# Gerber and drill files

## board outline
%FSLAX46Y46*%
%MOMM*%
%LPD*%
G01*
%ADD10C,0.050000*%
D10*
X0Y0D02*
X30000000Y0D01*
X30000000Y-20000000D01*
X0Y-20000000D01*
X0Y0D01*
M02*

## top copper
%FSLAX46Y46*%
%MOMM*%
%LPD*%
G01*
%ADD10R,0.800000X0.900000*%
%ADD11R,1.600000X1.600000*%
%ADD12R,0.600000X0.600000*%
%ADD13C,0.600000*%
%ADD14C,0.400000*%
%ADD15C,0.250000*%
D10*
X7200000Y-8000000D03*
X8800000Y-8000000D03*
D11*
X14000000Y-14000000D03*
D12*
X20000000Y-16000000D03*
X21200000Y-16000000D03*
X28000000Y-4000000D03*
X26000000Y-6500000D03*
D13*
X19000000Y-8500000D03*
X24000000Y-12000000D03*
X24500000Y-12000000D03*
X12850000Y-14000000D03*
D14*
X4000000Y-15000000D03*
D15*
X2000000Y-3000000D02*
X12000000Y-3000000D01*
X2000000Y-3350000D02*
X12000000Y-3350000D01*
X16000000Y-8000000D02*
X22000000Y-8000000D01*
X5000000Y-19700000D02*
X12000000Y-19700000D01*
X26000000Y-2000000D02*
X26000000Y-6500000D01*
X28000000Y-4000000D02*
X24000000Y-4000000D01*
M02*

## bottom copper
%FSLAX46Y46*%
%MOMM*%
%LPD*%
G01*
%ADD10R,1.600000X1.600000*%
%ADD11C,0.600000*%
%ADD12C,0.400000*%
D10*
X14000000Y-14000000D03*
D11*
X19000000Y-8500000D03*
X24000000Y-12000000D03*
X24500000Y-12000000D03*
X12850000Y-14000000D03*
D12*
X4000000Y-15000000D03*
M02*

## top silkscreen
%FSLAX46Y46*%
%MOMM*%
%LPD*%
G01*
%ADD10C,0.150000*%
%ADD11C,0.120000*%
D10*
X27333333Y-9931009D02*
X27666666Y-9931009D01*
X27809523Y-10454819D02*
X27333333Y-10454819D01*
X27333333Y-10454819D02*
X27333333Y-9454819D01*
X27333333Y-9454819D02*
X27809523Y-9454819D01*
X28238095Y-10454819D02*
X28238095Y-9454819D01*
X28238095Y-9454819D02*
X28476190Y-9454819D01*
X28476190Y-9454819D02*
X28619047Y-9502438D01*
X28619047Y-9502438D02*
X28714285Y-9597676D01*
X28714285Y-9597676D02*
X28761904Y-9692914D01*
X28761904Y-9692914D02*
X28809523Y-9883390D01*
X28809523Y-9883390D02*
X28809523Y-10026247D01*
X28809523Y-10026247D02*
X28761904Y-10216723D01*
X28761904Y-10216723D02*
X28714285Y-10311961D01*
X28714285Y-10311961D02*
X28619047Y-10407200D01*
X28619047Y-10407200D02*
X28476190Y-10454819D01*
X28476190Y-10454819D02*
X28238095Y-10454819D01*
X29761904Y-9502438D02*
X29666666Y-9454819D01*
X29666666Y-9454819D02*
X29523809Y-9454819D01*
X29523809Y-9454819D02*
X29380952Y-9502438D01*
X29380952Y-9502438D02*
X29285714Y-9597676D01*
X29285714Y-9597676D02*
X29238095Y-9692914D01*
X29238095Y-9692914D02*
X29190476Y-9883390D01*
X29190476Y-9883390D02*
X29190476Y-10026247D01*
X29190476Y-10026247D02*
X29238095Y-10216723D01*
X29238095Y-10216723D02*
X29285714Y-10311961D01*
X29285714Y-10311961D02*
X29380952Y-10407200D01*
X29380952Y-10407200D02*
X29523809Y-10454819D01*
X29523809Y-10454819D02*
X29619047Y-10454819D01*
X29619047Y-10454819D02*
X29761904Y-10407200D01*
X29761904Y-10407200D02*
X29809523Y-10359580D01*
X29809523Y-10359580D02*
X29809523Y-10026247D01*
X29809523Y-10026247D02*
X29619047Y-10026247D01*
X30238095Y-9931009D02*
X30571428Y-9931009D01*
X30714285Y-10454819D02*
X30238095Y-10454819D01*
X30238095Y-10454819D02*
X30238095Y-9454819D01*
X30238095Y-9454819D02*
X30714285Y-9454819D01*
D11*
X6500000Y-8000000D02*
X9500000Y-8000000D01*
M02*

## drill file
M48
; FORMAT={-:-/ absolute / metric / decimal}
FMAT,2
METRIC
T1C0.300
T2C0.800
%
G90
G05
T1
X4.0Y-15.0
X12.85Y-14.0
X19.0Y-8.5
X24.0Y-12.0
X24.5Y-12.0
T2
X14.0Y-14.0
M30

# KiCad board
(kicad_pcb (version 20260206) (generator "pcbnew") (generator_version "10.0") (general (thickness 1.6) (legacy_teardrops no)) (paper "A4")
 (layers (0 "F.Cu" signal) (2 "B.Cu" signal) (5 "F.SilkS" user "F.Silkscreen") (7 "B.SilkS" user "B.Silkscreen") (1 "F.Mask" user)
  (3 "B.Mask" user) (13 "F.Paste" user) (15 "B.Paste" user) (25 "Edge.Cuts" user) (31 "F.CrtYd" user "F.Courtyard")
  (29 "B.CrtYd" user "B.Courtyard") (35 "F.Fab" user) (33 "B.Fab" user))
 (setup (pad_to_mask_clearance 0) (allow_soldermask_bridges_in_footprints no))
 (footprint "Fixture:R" (layer "F.Cu") (at 8 8)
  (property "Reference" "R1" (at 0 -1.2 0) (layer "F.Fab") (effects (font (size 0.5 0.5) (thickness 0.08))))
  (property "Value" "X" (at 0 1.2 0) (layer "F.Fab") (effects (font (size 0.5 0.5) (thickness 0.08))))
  (pad "1" smd rect (at -0.8 0) (size 0.8 0.9) (layers "F.Cu" "F.Mask" "F.Paste") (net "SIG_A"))
  (pad "2" smd rect (at 0.8 0) (size 0.8 0.9) (layers "F.Cu" "F.Mask" "F.Paste") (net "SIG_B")))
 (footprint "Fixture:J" (layer "F.Cu") (at 14 14)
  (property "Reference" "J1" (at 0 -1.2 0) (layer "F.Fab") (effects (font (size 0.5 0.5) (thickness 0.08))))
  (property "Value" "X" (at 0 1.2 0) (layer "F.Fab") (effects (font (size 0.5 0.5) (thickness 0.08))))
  (pad "1" thru_hole rect (at 0 0) (size 1.6 1.6) (drill 0.8) (layers "*.Cu" "*.Mask") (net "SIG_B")))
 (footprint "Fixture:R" (layer "F.Cu") (at 20 16)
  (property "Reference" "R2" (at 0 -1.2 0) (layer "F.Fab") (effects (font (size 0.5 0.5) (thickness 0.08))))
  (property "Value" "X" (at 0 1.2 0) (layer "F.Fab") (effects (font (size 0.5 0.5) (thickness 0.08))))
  (pad "1" smd rect (at 0 0) (size 0.6 0.6) (layers "F.Cu" "F.Mask" "F.Paste")))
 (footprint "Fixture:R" (layer "F.Cu") (at 21.2 16)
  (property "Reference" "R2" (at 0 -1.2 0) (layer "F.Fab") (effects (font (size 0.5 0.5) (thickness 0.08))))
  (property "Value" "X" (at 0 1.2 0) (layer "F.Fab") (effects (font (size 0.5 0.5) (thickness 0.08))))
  (pad "1" smd rect (at 0 0) (size 0.6 0.6) (layers "F.Cu" "F.Mask" "F.Paste")))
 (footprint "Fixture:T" (layer "F.Cu") (at 28 4)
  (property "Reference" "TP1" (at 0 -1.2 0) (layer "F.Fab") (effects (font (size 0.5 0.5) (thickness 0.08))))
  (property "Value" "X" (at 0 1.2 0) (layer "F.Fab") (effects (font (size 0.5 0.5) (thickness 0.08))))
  (pad "1" smd rect (at 0 0) (size 0.6 0.6) (layers "F.Cu" "F.Mask" "F.Paste") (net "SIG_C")))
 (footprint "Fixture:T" (layer "F.Cu") (at 26 6.5)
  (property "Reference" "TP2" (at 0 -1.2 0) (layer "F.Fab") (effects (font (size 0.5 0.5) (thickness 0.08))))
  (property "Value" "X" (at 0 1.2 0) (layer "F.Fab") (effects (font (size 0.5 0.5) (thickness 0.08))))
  (pad "1" smd rect (at 0 0) (size 0.6 0.6) (layers "F.Cu" "F.Mask" "F.Paste") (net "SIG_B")))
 (gr_rect (start 0 0) (end 30 20) (stroke (width 0.05) (type default)) (fill no) (layer "Edge.Cuts"))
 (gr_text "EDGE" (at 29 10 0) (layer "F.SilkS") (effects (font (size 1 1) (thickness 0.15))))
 (gr_line (start 6.5 8) (end 9.5 8) (stroke (width 0.12) (type default)) (layer "F.SilkS"))
 (segment (start 2 3) (end 12 3) (width 0.25) (layer "F.Cu") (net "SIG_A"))
 (segment (start 2 3.35) (end 12 3.35) (width 0.25) (layer "F.Cu") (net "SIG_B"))
 (segment (start 16 8) (end 22 8) (width 0.25) (layer "F.Cu") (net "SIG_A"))
 (via (at 19 8.5) (size 0.6) (drill 0.3) (layers "F.Cu" "B.Cu") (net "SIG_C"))
 (via (at 24 12) (size 0.6) (drill 0.3) (layers "F.Cu" "B.Cu") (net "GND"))
 (via (at 24.5 12) (size 0.6) (drill 0.3) (layers "F.Cu" "B.Cu") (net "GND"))
 (segment (start 5 19.7) (end 12 19.7) (width 0.25) (layer "F.Cu") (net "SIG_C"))
 (segment (start 26 2) (end 26 6.5) (width 0.25) (layer "F.Cu") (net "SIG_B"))
 (segment (start 28 4) (end 24 4) (width 0.25) (layer "F.Cu") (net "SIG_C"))
 (via (at 12.85 14) (size 0.6) (drill 0.3) (layers "F.Cu" "B.Cu") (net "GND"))
 (via (at 4 15) (size 0.4) (drill 0.3) (layers "F.Cu" "B.Cu") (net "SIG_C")))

